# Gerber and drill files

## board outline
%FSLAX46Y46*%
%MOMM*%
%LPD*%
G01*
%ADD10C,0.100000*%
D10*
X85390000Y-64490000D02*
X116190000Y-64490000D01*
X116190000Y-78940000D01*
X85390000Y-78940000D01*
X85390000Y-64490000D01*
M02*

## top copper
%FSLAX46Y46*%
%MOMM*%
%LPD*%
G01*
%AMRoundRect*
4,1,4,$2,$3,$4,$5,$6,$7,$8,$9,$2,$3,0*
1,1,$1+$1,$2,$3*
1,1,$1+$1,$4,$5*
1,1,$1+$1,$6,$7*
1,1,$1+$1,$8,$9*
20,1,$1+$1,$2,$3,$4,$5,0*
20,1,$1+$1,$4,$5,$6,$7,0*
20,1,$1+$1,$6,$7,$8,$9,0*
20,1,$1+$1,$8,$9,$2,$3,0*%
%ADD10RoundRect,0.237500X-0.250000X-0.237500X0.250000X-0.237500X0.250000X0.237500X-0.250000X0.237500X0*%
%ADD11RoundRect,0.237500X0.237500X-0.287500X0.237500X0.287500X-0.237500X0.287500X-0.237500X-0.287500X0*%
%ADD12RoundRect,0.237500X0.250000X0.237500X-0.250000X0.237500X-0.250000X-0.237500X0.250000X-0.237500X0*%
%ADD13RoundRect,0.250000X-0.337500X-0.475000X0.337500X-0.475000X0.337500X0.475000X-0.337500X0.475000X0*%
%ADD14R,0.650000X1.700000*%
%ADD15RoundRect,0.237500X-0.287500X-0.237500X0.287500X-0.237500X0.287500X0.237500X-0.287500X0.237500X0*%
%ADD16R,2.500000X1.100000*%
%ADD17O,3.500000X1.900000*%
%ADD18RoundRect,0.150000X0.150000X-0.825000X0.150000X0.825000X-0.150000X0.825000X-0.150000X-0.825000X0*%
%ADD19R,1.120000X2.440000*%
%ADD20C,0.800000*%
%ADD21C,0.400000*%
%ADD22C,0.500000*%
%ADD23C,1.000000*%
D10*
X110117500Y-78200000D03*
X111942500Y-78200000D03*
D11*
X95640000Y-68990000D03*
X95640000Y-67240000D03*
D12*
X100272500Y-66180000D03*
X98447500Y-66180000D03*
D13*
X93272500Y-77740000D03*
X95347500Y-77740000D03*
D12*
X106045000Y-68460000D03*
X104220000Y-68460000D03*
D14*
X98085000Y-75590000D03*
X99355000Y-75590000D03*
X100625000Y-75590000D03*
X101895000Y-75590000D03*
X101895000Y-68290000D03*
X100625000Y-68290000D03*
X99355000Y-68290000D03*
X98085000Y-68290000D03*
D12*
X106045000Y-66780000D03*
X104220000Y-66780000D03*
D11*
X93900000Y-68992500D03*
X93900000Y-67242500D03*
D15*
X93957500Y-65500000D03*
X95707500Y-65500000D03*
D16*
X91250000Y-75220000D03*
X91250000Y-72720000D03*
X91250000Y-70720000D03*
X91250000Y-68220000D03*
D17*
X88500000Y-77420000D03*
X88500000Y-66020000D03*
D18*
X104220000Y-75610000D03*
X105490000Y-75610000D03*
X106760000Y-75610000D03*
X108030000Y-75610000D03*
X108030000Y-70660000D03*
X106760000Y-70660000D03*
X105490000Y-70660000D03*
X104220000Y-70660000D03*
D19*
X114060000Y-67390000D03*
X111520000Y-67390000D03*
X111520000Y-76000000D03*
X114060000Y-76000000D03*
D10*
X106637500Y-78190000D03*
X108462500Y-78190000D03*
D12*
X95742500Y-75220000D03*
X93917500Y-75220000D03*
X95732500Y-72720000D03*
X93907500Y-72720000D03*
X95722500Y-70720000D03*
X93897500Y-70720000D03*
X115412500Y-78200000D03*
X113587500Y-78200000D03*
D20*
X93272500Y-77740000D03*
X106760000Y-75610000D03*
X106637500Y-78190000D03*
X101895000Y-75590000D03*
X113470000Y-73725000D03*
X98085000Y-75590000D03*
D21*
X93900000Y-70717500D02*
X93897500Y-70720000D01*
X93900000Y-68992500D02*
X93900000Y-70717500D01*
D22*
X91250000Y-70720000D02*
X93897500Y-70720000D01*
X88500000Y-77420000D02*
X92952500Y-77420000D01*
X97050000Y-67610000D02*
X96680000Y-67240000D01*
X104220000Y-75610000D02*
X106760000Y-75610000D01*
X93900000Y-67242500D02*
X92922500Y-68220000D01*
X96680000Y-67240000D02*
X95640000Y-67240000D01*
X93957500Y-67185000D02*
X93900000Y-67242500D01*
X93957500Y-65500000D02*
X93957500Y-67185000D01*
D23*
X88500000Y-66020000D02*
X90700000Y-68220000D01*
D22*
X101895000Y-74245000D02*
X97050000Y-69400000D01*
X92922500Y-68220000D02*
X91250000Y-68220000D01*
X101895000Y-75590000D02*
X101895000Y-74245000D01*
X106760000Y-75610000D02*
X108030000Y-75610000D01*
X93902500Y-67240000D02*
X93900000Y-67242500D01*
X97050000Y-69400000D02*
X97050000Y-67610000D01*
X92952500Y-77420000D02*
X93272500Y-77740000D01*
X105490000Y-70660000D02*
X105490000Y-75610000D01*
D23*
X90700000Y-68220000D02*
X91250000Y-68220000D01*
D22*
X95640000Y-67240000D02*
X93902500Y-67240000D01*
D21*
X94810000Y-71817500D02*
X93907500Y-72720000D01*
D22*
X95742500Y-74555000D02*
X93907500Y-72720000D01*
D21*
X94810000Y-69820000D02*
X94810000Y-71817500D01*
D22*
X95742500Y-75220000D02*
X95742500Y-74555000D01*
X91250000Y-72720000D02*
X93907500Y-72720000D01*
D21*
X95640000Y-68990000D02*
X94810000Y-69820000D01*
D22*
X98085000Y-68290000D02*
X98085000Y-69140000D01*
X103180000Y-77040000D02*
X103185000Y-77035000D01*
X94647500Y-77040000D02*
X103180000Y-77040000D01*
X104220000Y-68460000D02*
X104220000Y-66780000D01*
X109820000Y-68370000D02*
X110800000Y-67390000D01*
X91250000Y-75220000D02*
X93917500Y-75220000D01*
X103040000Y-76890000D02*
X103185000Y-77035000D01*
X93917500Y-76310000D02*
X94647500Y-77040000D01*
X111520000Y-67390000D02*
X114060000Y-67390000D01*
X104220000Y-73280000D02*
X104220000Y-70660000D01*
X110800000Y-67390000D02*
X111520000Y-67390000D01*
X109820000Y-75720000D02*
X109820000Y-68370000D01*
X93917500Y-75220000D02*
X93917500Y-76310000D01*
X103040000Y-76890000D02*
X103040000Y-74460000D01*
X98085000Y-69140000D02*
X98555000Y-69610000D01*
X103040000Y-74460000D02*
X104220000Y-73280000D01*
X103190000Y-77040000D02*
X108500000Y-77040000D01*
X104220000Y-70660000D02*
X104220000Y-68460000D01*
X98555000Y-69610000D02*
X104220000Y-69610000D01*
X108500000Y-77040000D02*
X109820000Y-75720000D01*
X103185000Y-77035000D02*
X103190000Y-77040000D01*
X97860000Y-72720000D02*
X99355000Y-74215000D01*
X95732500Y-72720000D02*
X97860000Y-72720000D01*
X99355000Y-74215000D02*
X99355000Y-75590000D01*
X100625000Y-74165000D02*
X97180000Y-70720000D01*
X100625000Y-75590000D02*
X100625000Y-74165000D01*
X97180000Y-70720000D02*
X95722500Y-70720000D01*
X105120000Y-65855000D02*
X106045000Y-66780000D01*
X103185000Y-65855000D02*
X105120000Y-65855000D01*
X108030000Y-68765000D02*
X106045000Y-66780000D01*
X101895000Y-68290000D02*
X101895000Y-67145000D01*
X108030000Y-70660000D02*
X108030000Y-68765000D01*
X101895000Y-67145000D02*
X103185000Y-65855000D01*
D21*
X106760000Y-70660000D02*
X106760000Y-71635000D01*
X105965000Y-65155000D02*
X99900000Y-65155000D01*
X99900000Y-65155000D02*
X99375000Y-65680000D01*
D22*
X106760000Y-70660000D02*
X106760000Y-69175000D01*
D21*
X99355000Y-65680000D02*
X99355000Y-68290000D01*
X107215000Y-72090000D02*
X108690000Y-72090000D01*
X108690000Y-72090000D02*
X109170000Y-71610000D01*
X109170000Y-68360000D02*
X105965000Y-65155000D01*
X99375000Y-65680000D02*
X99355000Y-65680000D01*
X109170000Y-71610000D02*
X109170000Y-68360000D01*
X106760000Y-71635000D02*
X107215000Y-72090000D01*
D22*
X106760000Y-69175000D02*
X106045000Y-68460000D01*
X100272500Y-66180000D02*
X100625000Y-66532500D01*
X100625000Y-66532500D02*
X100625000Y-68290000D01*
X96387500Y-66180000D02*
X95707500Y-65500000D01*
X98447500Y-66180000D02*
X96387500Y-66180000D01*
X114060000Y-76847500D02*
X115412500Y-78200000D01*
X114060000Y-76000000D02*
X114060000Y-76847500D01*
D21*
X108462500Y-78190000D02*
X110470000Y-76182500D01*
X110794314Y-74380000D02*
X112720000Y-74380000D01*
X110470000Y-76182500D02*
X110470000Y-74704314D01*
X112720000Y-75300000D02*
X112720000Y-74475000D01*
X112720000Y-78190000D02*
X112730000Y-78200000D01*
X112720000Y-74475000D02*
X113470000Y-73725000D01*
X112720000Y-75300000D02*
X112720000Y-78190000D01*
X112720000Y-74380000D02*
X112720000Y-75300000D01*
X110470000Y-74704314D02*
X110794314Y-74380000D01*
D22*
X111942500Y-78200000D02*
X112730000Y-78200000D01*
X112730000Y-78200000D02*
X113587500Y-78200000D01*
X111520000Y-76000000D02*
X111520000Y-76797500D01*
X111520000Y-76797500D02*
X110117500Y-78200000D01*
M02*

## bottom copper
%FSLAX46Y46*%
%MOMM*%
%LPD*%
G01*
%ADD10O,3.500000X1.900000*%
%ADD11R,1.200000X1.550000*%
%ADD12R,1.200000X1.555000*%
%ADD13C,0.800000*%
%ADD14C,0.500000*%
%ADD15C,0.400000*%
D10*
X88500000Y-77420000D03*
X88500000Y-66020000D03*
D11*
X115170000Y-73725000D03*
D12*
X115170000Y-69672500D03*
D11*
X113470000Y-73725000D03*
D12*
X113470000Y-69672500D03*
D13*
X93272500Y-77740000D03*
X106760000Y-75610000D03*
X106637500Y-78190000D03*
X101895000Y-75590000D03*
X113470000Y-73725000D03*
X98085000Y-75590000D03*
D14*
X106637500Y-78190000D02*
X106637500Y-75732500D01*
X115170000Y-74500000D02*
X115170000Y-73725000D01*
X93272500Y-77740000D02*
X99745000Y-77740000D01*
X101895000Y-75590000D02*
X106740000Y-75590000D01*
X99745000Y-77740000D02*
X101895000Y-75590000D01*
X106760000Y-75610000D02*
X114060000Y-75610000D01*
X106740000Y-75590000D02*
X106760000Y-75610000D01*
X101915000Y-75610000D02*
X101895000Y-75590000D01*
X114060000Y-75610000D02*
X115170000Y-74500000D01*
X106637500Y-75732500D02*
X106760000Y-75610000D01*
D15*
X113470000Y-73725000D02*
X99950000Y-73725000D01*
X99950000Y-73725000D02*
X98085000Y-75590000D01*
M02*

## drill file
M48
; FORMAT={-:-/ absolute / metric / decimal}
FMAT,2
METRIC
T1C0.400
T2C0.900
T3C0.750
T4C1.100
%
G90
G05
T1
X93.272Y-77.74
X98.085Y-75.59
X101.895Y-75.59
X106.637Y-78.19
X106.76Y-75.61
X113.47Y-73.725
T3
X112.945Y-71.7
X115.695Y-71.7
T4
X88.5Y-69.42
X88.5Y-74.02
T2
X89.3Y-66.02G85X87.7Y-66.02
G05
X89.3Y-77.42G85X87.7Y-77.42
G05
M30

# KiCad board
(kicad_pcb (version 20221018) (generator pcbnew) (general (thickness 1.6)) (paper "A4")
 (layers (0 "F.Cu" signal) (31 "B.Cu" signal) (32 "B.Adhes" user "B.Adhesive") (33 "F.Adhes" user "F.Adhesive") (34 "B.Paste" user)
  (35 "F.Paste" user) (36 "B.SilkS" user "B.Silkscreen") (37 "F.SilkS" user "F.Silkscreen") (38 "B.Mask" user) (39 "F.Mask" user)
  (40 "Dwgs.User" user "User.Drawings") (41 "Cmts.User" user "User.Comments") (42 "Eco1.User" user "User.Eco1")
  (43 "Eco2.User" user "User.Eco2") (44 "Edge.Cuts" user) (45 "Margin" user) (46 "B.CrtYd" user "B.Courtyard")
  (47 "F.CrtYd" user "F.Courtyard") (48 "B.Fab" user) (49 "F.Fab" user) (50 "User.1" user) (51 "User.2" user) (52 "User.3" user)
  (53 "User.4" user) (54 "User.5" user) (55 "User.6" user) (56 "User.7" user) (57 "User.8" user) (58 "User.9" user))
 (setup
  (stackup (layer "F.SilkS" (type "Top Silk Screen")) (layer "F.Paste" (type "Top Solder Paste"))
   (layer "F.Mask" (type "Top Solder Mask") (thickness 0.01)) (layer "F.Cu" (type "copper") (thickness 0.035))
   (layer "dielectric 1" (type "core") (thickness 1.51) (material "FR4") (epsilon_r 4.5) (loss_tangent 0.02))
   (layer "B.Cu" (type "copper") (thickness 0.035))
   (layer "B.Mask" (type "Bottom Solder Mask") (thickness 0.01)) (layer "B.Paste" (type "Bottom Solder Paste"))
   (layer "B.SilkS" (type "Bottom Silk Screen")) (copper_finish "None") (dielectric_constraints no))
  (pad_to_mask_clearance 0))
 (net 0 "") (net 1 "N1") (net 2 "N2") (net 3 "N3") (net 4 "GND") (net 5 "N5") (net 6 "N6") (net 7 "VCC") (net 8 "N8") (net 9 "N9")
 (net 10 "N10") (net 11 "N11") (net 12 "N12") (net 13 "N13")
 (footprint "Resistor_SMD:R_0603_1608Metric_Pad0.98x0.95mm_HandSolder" (layer "F.Cu") (at 111.03 78.2)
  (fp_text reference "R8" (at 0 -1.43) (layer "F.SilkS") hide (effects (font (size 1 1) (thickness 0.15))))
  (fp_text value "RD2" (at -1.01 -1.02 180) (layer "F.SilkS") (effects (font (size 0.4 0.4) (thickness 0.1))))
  (pad "1" smd roundrect (at -0.9125 0) (size 0.975 0.95) (layers "F.Cu" "F.Paste" "F.Mask") (roundrect_rratio 0.25) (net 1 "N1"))
  (pad "2" smd roundrect (at 0.9125 0) (size 0.975 0.95) (layers "F.Cu" "F.Paste" "F.Mask") (roundrect_rratio 0.25) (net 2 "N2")))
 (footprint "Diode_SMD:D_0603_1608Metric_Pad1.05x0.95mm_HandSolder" (layer "F.Cu") (at 95.64 68.115 90)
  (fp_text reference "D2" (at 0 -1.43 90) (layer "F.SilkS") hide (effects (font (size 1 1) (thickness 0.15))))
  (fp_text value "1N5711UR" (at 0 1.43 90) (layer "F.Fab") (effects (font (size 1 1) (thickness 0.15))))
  (pad "1" smd roundrect (at -0.875 0 90) (size 1.05 0.95) (layers "F.Cu" "F.Paste" "F.Mask") (roundrect_rratio 0.25) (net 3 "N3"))
  (pad "2" smd roundrect (at 0.875 0 90) (size 1.05 0.95) (layers "F.Cu" "F.Paste" "F.Mask") (roundrect_rratio 0.25) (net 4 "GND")))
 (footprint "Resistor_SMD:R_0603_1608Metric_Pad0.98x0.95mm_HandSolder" (layer "F.Cu") (at 99.36 66.18 180)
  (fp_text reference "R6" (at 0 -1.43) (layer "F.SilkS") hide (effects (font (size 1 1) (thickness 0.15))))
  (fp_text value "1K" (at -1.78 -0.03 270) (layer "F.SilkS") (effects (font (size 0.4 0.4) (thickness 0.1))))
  (pad "1" smd roundrect (at -0.9125 0 180) (size 0.975 0.95) (layers "F.Cu" "F.Paste" "F.Mask") (roundrect_rratio 0.25) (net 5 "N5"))
  (pad "2" smd roundrect (at 0.9125 0 180) (size 0.975 0.95) (layers "F.Cu" "F.Paste" "F.Mask") (roundrect_rratio 0.25) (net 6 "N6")))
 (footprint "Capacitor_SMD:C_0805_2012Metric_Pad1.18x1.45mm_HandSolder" (layer "F.Cu") (at 94.31 77.74)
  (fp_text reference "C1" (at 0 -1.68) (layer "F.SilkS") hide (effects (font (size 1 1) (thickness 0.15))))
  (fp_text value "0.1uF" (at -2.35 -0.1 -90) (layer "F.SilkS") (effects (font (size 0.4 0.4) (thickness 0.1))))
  (pad "1" smd roundrect (at -1.0375 0) (size 1.175 1.45) (layers "F.Cu" "F.Paste" "F.Mask") (roundrect_rratio 0.212766) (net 4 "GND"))
  (pad "2" smd roundrect (at 1.0375 0) (size 1.175 1.45) (layers "F.Cu" "F.Paste" "F.Mask") (roundrect_rratio 0.212766) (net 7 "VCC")))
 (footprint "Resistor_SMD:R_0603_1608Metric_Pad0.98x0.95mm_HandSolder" (layer "F.Cu") (at 105.1325 68.46 180)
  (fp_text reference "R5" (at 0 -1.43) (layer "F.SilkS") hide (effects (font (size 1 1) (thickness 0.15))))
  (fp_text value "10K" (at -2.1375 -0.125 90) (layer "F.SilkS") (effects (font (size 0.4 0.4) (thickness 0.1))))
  (pad "1" smd roundrect (at -0.9125 0 180) (size 0.975 0.95) (layers "F.Cu" "F.Paste" "F.Mask") (roundrect_rratio 0.25) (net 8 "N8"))
  (pad "2" smd roundrect (at 0.9125 0 180) (size 0.975 0.95) (layers "F.Cu" "F.Paste" "F.Mask") (roundrect_rratio 0.25) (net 7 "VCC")))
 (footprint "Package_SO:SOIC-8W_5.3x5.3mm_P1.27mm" (layer "F.Cu") (at 99.99 71.94 90)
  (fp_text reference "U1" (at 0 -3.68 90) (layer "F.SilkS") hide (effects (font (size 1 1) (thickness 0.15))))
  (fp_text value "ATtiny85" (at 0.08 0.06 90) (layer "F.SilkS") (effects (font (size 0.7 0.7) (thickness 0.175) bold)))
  (pad "1" smd rect (at -3.65 -1.905 90) (size 1.7 0.65) (layers "F.Cu" "F.Paste" "F.Mask") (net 2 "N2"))
  (pad "2" smd rect (at -3.65 -0.635 90) (size 1.7 0.65) (layers "F.Cu" "F.Paste" "F.Mask") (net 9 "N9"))
  (pad "3" smd rect (at -3.65 0.635 90) (size 1.7 0.65) (layers "F.Cu" "F.Paste" "F.Mask") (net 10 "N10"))
  (pad "4" smd rect (at -3.65 1.905 90) (size 1.7 0.65) (layers "F.Cu" "F.Paste" "F.Mask") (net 4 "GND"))
  (pad "5" smd rect (at 3.65 1.905 90) (size 1.7 0.65) (layers "F.Cu" "F.Paste" "F.Mask") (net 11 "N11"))
  (pad "6" smd rect (at 3.65 0.635 90) (size 1.7 0.65) (layers "F.Cu" "F.Paste" "F.Mask") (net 5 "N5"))
  (pad "7" smd rect (at 3.65 -0.635 90) (size 1.7 0.65) (layers "F.Cu" "F.Paste" "F.Mask") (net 8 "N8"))
  (pad "8" smd rect (at 3.65 -1.905 90) (size 1.7 0.65) (layers "F.Cu" "F.Paste" "F.Mask") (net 7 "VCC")))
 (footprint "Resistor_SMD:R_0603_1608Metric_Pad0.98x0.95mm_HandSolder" (layer "F.Cu") (at 105.1325 66.78 180)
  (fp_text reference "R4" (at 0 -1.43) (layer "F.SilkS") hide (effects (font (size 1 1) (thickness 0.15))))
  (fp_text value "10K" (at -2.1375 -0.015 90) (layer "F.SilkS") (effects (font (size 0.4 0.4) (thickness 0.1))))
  (pad "1" smd roundrect (at -0.9125 0 180) (size 0.975 0.95) (layers "F.Cu" "F.Paste" "F.Mask") (roundrect_rratio 0.25) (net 11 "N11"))
  (pad "2" smd roundrect (at 0.9125 0 180) (size 0.975 0.95) (layers "F.Cu" "F.Paste" "F.Mask") (roundrect_rratio 0.25) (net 7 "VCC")))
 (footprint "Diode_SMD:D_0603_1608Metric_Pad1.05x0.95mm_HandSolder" (layer "F.Cu") (at 93.9 68.1175 90)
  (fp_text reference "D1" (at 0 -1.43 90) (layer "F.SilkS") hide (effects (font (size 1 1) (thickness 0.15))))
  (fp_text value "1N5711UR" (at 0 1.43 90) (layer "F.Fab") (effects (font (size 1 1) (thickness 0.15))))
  (pad "1" smd roundrect (at -0.875 0 90) (size 1.05 0.95) (layers "F.Cu" "F.Paste" "F.Mask") (roundrect_rratio 0.25) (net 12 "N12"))
  (pad "2" smd roundrect (at 0.875 0 90) (size 1.05 0.95) (layers "F.Cu" "F.Paste" "F.Mask") (roundrect_rratio 0.25) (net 4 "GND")))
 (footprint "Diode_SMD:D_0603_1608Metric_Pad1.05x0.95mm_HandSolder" (layer "F.Cu") (at 94.8325 65.5)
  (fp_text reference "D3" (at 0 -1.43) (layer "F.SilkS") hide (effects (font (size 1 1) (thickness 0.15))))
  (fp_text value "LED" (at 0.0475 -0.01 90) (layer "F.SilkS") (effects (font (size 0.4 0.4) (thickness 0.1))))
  (pad "1" smd roundrect (at -0.875 0) (size 1.05 0.95) (layers "F.Cu" "F.Paste" "F.Mask") (roundrect_rratio 0.25) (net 4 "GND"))
  (pad "2" smd roundrect (at 0.875 0) (size 1.05 0.95) (layers "F.Cu" "F.Paste" "F.Mask") (roundrect_rratio 0.25) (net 6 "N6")))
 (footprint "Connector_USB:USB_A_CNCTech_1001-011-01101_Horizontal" (layer "F.Cu") (at 81.6 71.72 180)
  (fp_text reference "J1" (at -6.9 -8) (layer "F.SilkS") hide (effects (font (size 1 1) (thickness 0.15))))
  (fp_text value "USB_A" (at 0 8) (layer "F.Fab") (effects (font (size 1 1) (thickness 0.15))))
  (pad "" np_thru_hole circle (at -6.9 -2.3 180) (size 1.1 1.1) (drill 1.1) (layers "*.Cu" "*.Mask"))
  (pad "" np_thru_hole circle (at -6.9 2.3 180) (size 1.1 1.1) (drill 1.1) (layers "*.Cu" "*.Mask"))
  (pad "1" smd rect (at -9.65 -3.5 180) (size 2.5 1.1) (layers "F.Cu" "F.Paste" "F.Mask") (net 7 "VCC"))
  (pad "2" smd rect (at -9.65 -1 180) (size 2.5 1.1) (layers "F.Cu" "F.Paste" "F.Mask") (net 3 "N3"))
  (pad "3" smd rect (at -9.65 1 180) (size 2.5 1.1) (layers "F.Cu" "F.Paste" "F.Mask") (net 12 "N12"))
  (pad "4" smd rect (at -9.65 3.5 180) (size 2.5 1.1) (layers "F.Cu" "F.Paste" "F.Mask") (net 4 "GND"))
  (pad "5" thru_hole oval (at -6.9 -5.7 180) (size 3.5 1.9) (drill oval 2.5 0.9) (layers "*.Cu" "*.Mask") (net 4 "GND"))
  (pad "5" thru_hole oval (at -6.9 5.7 180) (size 3.5 1.9) (drill oval 2.5 0.9) (layers "*.Cu" "*.Mask") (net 4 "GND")))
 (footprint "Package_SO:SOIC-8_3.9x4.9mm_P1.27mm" (layer "F.Cu") (at 106.125 73.135 90)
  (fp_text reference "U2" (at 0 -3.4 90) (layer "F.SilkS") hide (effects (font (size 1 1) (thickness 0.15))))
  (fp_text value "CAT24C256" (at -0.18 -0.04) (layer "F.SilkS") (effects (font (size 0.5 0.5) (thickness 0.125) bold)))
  (pad "1" smd roundrect (at -2.475 -1.905 90) (size 1.95 0.6) (layers "F.Cu" "F.Paste" "F.Mask") (roundrect_rratio 0.25) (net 4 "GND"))
  (pad "2" smd roundrect (at -2.475 -0.635 90) (size 1.95 0.6) (layers "F.Cu" "F.Paste" "F.Mask") (roundrect_rratio 0.25) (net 4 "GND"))
  (pad "3" smd roundrect (at -2.475 0.635 90) (size 1.95 0.6) (layers "F.Cu" "F.Paste" "F.Mask") (roundrect_rratio 0.25) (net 4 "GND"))
  (pad "4" smd roundrect (at -2.475 1.905 90) (size 1.95 0.6) (layers "F.Cu" "F.Paste" "F.Mask") (roundrect_rratio 0.25) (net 4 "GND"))
  (pad "5" smd roundrect (at 2.475 1.905 90) (size 1.95 0.6) (layers "F.Cu" "F.Paste" "F.Mask") (roundrect_rratio 0.25) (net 11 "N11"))
  (pad "6" smd roundrect (at 2.475 0.635 90) (size 1.95 0.6) (layers "F.Cu" "F.Paste" "F.Mask") (roundrect_rratio 0.25) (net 8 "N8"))
  (pad "7" smd roundrect (at 2.475 -0.635 90) (size 1.95 0.6) (layers "F.Cu" "F.Paste" "F.Mask") (roundrect_rratio 0.25) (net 4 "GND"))
  (pad "8" smd roundrect (at 2.475 -1.905 90) (size 1.95 0.6) (layers "F.Cu" "F.Paste" "F.Mask") (roundrect_rratio 0.25) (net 7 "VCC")))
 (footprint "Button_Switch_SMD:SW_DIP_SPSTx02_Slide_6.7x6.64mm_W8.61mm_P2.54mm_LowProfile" (layer "F.Cu") (at 112.79 71.695 -90)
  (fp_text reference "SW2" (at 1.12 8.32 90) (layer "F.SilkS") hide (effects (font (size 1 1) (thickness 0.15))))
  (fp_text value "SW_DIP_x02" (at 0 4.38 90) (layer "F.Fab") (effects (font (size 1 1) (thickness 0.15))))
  (pad "1" smd rect (at -4.305 -1.27 270) (size 2.44 1.12) (layers "F.Cu" "F.Paste" "F.Mask") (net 7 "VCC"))
  (pad "2" smd rect (at -4.305 1.27 270) (size 2.44 1.12) (layers "F.Cu" "F.Paste" "F.Mask") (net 7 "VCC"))
  (pad "3" smd rect (at 4.305 1.27 270) (size 2.44 1.12) (layers "F.Cu" "F.Paste" "F.Mask") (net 1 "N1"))
  (pad "4" smd rect (at 4.305 -1.27 270) (size 2.44 1.12) (layers "F.Cu" "F.Paste" "F.Mask") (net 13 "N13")))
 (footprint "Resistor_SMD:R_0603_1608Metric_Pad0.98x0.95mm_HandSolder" (layer "F.Cu") (at 107.55 78.19)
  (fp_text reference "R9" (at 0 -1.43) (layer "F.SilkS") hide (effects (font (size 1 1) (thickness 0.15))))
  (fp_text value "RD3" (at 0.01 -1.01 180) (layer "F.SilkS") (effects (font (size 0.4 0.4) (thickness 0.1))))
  (pad "1" smd roundrect (at -0.9125 0) (size 0.975 0.95) (layers "F.Cu" "F.Paste" "F.Mask") (roundrect_rratio 0.25) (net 4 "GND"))
  (pad "2" smd roundrect (at 0.9125 0) (size 0.975 0.95) (layers "F.Cu" "F.Paste" "F.Mask") (roundrect_rratio 0.25) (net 2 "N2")))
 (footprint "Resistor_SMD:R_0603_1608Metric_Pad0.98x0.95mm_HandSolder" (layer "F.Cu") (at 94.83 75.22 180)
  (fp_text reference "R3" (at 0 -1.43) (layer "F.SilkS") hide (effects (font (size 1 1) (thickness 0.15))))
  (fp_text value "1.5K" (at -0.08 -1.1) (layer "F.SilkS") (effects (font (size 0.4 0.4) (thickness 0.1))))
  (pad "1" smd roundrect (at -0.9125 0 180) (size 0.975 0.95) (layers "F.Cu" "F.Paste" "F.Mask") (roundrect_rratio 0.25) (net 3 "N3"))
  (pad "2" smd roundrect (at 0.9125 0 180) (size 0.975 0.95) (layers "F.Cu" "F.Paste" "F.Mask") (roundrect_rratio 0.25) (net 7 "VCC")))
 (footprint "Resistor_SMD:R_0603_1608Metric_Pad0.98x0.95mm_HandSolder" (layer "F.Cu") (at 94.82 72.72 180)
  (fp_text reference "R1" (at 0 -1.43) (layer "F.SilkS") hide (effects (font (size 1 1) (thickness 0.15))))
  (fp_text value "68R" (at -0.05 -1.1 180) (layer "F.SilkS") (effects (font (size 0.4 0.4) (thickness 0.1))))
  (pad "1" smd roundrect (at -0.9125 0 180) (size 0.975 0.95) (layers "F.Cu" "F.Paste" "F.Mask") (roundrect_rratio 0.25) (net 9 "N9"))
  (pad "2" smd roundrect (at 0.9125 0 180) (size 0.975 0.95) (layers "F.Cu" "F.Paste" "F.Mask") (roundrect_rratio 0.25) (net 3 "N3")))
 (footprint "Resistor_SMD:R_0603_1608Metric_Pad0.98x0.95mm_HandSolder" (layer "F.Cu") (at 94.81 70.72 180)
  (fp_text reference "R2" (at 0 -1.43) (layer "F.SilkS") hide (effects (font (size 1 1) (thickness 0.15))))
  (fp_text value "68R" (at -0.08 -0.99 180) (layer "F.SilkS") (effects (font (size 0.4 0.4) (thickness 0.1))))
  (pad "1" smd roundrect (at -0.9125 0 180) (size 0.975 0.95) (layers "F.Cu" "F.Paste" "F.Mask") (roundrect_rratio 0.25) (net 10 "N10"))
  (pad "2" smd roundrect (at 0.9125 0 180) (size 0.975 0.95) (layers "F.Cu" "F.Paste" "F.Mask") (roundrect_rratio 0.25) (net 12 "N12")))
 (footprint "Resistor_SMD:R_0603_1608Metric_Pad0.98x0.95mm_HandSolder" (layer "F.Cu") (at 114.5 78.2 180)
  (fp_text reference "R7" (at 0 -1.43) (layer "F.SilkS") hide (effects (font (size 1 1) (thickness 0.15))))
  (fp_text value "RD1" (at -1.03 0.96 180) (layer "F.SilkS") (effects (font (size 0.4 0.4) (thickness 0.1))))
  (pad "1" smd roundrect (at -0.9125 0 180) (size 0.975 0.95) (layers "F.Cu" "F.Paste" "F.Mask") (roundrect_rratio 0.25) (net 13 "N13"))
  (pad "2" smd roundrect (at 0.9125 0 180) (size 0.975 0.95) (layers "F.Cu" "F.Paste" "F.Mask") (roundrect_rratio 0.25) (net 2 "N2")))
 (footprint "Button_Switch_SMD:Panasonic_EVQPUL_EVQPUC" (layer "B.Cu") (at 114.32 71.7 90)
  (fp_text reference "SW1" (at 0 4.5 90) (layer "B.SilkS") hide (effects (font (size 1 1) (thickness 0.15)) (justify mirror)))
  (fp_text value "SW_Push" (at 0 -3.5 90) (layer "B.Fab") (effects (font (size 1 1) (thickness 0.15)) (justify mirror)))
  (pad "" np_thru_hole circle (at 0 -1.375 270) (size 0.75 0.75) (drill 0.75) (layers "F&B.Cu" "*.Mask"))
  (pad "" np_thru_hole circle (at 0 1.375 270) (size 0.75 0.75) (drill 0.75) (layers "F&B.Cu" "*.Mask"))
  (pad "1" smd rect (at -2.025 0.85 270) (size 1.55 1.2) (layers "B.Cu" "B.Paste" "B.Mask") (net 4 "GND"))
  (pad "1" smd rect (at 2.0275 0.85 270) (size 1.555 1.2) (layers "B.Cu" "B.Paste" "B.Mask") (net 4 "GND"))
  (pad "2" smd rect (at -2.025 -0.85 270) (size 1.55 1.2) (layers "B.Cu" "B.Paste" "B.Mask") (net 2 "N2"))
  (pad "2" smd rect (at 2.0275 -0.85 270) (size 1.555 1.2) (layers "B.Cu" "B.Paste" "B.Mask") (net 2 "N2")))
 (gr_rect (start 85.39 64.49) (end 116.19 78.94) (stroke (width 0.1) (type default)) (fill none) (layer "Edge.Cuts"))
 (segment (start 93.9 70.7175) (end 93.8975 70.72) (width 0.4) (layer "F.Cu") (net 12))
 (segment (start 93.9 68.9925) (end 93.9 70.7175) (width 0.4) (layer "F.Cu") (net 12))
 (segment (start 91.25 70.72) (end 93.8975 70.72) (width 0.5) (layer "F.Cu") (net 12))
 (segment (start 88.5 77.42) (end 92.9525 77.42) (width 0.5) (layer "F.Cu") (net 4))
 (segment (start 97.05 67.61) (end 96.68 67.24) (width 0.5) (layer "F.Cu") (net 4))
 (segment (start 104.22 75.61) (end 106.76 75.61) (width 0.5) (layer "F.Cu") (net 4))
 (segment (start 93.9 67.2425) (end 92.9225 68.22) (width 0.5) (layer "F.Cu") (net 4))
 (segment (start 96.68 67.24) (end 95.64 67.24) (width 0.5) (layer "F.Cu") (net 4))
 (segment (start 93.9575 67.185) (end 93.9 67.2425) (width 0.5) (layer "F.Cu") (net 4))
 (segment (start 93.9575 65.5) (end 93.9575 67.185) (width 0.5) (layer "F.Cu") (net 4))
 (segment (start 88.5 66.02) (end 90.7 68.22) (width 1) (layer "F.Cu") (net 4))
 (segment (start 101.895 74.245) (end 97.05 69.4) (width 0.5) (layer "F.Cu") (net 4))
 (segment (start 92.9225 68.22) (end 91.25 68.22) (width 0.5) (layer "F.Cu") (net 4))
 (segment (start 101.895 75.59) (end 101.895 74.245) (width 0.5) (layer "F.Cu") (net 4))
 (segment (start 106.76 75.61) (end 108.03 75.61) (width 0.5) (layer "F.Cu") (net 4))
 (segment (start 93.9025 67.24) (end 93.9 67.2425) (width 0.5) (layer "F.Cu") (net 4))
 (segment (start 97.05 69.4) (end 97.05 67.61) (width 0.5) (layer "F.Cu") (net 4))
 (segment (start 92.9525 77.42) (end 93.2725 77.74) (width 0.5) (layer "F.Cu") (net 4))
 (segment (start 105.49 70.66) (end 105.49 75.61) (width 0.5) (layer "F.Cu") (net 4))
 (segment (start 90.7 68.22) (end 91.25 68.22) (width 1) (layer "F.Cu") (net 4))
 (segment (start 95.64 67.24) (end 93.9025 67.24) (width 0.5) (layer "F.Cu") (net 4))
 (via (at 93.2725 77.74) (size 0.8) (drill 0.4) (layers "F.Cu" "B.Cu") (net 4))
 (via (at 106.76 75.61) (size 0.8) (drill 0.4) (layers "F.Cu" "B.Cu") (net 4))
 (via (at 106.6375 78.19) (size 0.8) (drill 0.4) (layers "F.Cu" "B.Cu") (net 4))
 (via (at 101.895 75.59) (size 0.8) (drill 0.4) (layers "F.Cu" "B.Cu") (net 4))
 (segment (start 106.6375 78.19) (end 106.6375 75.7325) (width 0.5) (layer "B.Cu") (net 4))
 (segment (start 115.17 74.5) (end 115.17 73.725) (width 0.5) (layer "B.Cu") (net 4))
 (segment (start 93.2725 77.74) (end 99.745 77.74) (width 0.5) (layer "B.Cu") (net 4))
 (segment (start 101.895 75.59) (end 106.74 75.59) (width 0.5) (layer "B.Cu") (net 4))
 (segment (start 99.745 77.74) (end 101.895 75.59) (width 0.5) (layer "B.Cu") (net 4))
 (segment (start 106.76 75.61) (end 114.06 75.61) (width 0.5) (layer "B.Cu") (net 4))
 (segment (start 106.74 75.59) (end 106.76 75.61) (width 0.5) (layer "B.Cu") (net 4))
 (segment (start 101.915 75.61) (end 101.895 75.59) (width 0.5) (layer "B.Cu") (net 4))
 (segment (start 114.06 75.61) (end 115.17 74.5) (width 0.5) (layer "B.Cu") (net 4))
 (segment (start 106.6375 75.7325) (end 106.76 75.61) (width 0.5) (layer "B.Cu") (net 4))
 (segment (start 94.81 71.8175) (end 93.9075 72.72) (width 0.4) (layer "F.Cu") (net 3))
 (segment (start 95.7425 74.555) (end 93.9075 72.72) (width 0.5) (layer "F.Cu") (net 3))
 (segment (start 94.81 69.82) (end 94.81 71.8175) (width 0.4) (layer "F.Cu") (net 3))
 (segment (start 95.7425 75.22) (end 95.7425 74.555) (width 0.5) (layer "F.Cu") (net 3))
 (segment (start 91.25 72.72) (end 93.9075 72.72) (width 0.5) (layer "F.Cu") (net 3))
 (segment (start 95.64 68.99) (end 94.81 69.82) (width 0.4) (layer "F.Cu") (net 3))
 (segment (start 98.085 68.29) (end 98.085 69.14) (width 0.5) (layer "F.Cu") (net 7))
 (segment (start 103.18 77.04) (end 103.185 77.035) (width 0.5) (layer "F.Cu") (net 7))
 (segment (start 94.6475 77.04) (end 103.18 77.04) (width 0.5) (layer "F.Cu") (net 7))
 (segment (start 104.22 68.46) (end 104.22 66.78) (width 0.5) (layer "F.Cu") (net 7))
 (segment (start 109.82 68.37) (end 110.8 67.39) (width 0.5) (layer "F.Cu") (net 7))
 (segment (start 91.25 75.22) (end 93.9175 75.22) (width 0.5) (layer "F.Cu") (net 7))
 (segment (start 103.04 76.89) (end 103.185 77.035) (width 0.5) (layer "F.Cu") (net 7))
 (segment (start 93.9175 76.31) (end 94.6475 77.04) (width 0.5) (layer "F.Cu") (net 7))
 (segment (start 111.52 67.39) (end 114.06 67.39) (width 0.5) (layer "F.Cu") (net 7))
 (segment (start 104.22 73.28) (end 104.22 70.66) (width 0.5) (layer "F.Cu") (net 7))
 (segment (start 110.8 67.39) (end 111.52 67.39) (width 0.5) (layer "F.Cu") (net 7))
 (segment (start 109.82 75.72) (end 109.82 68.37) (width 0.5) (layer "F.Cu") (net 7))
 (segment (start 93.9175 75.22) (end 93.9175 76.31) (width 0.5) (layer "F.Cu") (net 7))
 (segment (start 103.04 76.89) (end 103.04 74.46) (width 0.5) (layer "F.Cu") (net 7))
 (segment (start 98.085 69.14) (end 98.555 69.61) (width 0.5) (layer "F.Cu") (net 7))
 (segment (start 103.04 74.46) (end 104.22 73.28) (width 0.5) (layer "F.Cu") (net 7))
 (segment (start 103.19 77.04) (end 108.5 77.04) (width 0.5) (layer "F.Cu") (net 7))
 (segment (start 104.22 70.66) (end 104.22 68.46) (width 0.5) (layer "F.Cu") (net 7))
 (segment (start 98.555 69.61) (end 104.22 69.61) (width 0.5) (layer "F.Cu") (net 7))
 (segment (start 108.5 77.04) (end 109.82 75.72) (width 0.5) (layer "F.Cu") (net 7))
 (segment (start 103.185 77.035) (end 103.19 77.04) (width 0.5) (layer "F.Cu") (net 7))
 (segment (start 97.86 72.72) (end 99.355 74.215) (width 0.5) (layer "F.Cu") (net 9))
 (segment (start 95.7325 72.72) (end 97.86 72.72) (width 0.5) (layer "F.Cu") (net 9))
 (segment (start 99.355 74.215) (end 99.355 75.59) (width 0.5) (layer "F.Cu") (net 9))
 (segment (start 100.625 74.165) (end 97.18 70.72) (width 0.5) (layer "F.Cu") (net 10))
 (segment (start 100.625 75.59) (end 100.625 74.165) (width 0.5) (layer "F.Cu") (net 10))
 (segment (start 97.18 70.72) (end 95.7225 70.72) (width 0.5) (layer "F.Cu") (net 10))
 (segment (start 105.12 65.855) (end 106.045 66.78) (width 0.5) (layer "F.Cu") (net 11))
 (segment (start 103.185 65.855) (end 105.12 65.855) (width 0.5) (layer "F.Cu") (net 11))
 (segment (start 108.03 68.765) (end 106.045 66.78) (width 0.5) (layer "F.Cu") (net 11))
 (segment (start 101.895 68.29) (end 101.895 67.145) (width 0.5) (layer "F.Cu") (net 11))
 (segment (start 108.03 70.66) (end 108.03 68.765) (width 0.5) (layer "F.Cu") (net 11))
 (segment (start 101.895 67.145) (end 103.185 65.855) (width 0.5) (layer "F.Cu") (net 11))
 (segment (start 106.76 70.66) (end 106.76 71.635) (width 0.4) (layer "F.Cu") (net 8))
 (segment (start 105.965 65.155) (end 99.9 65.155) (width 0.4) (layer "F.Cu") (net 8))
 (segment (start 99.9 65.155) (end 99.375 65.68) (width 0.4) (layer "F.Cu") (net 8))
 (segment (start 106.76 70.66) (end 106.76 69.175) (width 0.5) (layer "F.Cu") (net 8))
 (segment (start 99.355 65.68) (end 99.355 68.29) (width 0.4) (layer "F.Cu") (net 8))
 (segment (start 107.215 72.09) (end 108.69 72.09) (width 0.4) (layer "F.Cu") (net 8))
 (segment (start 108.69 72.09) (end 109.17 71.61) (width 0.4) (layer "F.Cu") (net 8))
 (segment (start 109.17 68.36) (end 105.965 65.155) (width 0.4) (layer "F.Cu") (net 8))
 (segment (start 99.375 65.68) (end 99.355 65.68) (width 0.4) (layer "F.Cu") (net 8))
 (segment (start 109.17 71.61) (end 109.17 68.36) (width 0.4) (layer "F.Cu") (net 8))
 (segment (start 106.76 71.635) (end 107.215 72.09) (width 0.4) (layer "F.Cu") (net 8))
 (segment (start 106.76 69.175) (end 106.045 68.46) (width 0.5) (layer "F.Cu") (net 8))
 (segment (start 100.2725 66.18) (end 100.625 66.5325) (width 0.5) (layer "F.Cu") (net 5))
 (segment (start 100.625 66.5325) (end 100.625 68.29) (width 0.5) (layer "F.Cu") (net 5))
 (segment (start 96.3875 66.18) (end 95.7075 65.5) (width 0.5) (layer "F.Cu") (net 6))
 (segment (start 98.4475 66.18) (end 96.3875 66.18) (width 0.5) (layer "F.Cu") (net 6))
 (segment (start 114.06 76.8475) (end 115.4125 78.2) (width 0.5) (layer "F.Cu") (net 13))
 (segment (start 114.06 76) (end 114.06 76.8475) (width 0.5) (layer "F.Cu") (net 13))
 (segment (start 108.4625 78.19) (end 110.47 76.1825) (width 0.4) (layer "F.Cu") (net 2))
 (segment (start 110.794314 74.38) (end 112.72 74.38) (width 0.4) (layer "F.Cu") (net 2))
 (segment (start 110.47 76.1825) (end 110.47 74.704314) (width 0.4) (layer "F.Cu") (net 2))
 (segment (start 112.72 75.3) (end 112.72 74.475) (width 0.4) (layer "F.Cu") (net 2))
 (segment (start 112.72 78.19) (end 112.73 78.2) (width 0.4) (layer "F.Cu") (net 2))
 (segment (start 112.72 74.475) (end 113.47 73.725) (width 0.4) (layer "F.Cu") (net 2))
 (segment (start 112.72 75.3) (end 112.72 78.19) (width 0.4) (layer "F.Cu") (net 2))
 (segment (start 112.72 74.38) (end 112.72 75.3) (width 0.4) (layer "F.Cu") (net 2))
 (segment (start 110.47 74.704314) (end 110.794314 74.38) (width 0.4) (layer "F.Cu") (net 2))
 (segment (start 111.9425 78.2) (end 112.73 78.2) (width 0.5) (layer "F.Cu") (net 2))
 (segment (start 112.73 78.2) (end 113.5875 78.2) (width 0.5) (layer "F.Cu") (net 2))
 (via (at 113.47 73.725) (size 0.8) (drill 0.4) (layers "F.Cu" "B.Cu") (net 2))
 (via (at 98.085 75.59) (size 0.8) (drill 0.4) (layers "F.Cu" "B.Cu") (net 2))
 (segment (start 113.47 73.725) (end 99.95 73.725) (width 0.4) (layer "B.Cu") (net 2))
 (segment (start 99.95 73.725) (end 98.085 75.59) (width 0.4) (layer "B.Cu") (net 2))
 (segment (start 111.52 76) (end 111.52 76.7975) (width 0.5) (layer "F.Cu") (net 1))
 (segment (start 111.52 76.7975) (end 110.1175 78.2) (width 0.5) (layer "F.Cu") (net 1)))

